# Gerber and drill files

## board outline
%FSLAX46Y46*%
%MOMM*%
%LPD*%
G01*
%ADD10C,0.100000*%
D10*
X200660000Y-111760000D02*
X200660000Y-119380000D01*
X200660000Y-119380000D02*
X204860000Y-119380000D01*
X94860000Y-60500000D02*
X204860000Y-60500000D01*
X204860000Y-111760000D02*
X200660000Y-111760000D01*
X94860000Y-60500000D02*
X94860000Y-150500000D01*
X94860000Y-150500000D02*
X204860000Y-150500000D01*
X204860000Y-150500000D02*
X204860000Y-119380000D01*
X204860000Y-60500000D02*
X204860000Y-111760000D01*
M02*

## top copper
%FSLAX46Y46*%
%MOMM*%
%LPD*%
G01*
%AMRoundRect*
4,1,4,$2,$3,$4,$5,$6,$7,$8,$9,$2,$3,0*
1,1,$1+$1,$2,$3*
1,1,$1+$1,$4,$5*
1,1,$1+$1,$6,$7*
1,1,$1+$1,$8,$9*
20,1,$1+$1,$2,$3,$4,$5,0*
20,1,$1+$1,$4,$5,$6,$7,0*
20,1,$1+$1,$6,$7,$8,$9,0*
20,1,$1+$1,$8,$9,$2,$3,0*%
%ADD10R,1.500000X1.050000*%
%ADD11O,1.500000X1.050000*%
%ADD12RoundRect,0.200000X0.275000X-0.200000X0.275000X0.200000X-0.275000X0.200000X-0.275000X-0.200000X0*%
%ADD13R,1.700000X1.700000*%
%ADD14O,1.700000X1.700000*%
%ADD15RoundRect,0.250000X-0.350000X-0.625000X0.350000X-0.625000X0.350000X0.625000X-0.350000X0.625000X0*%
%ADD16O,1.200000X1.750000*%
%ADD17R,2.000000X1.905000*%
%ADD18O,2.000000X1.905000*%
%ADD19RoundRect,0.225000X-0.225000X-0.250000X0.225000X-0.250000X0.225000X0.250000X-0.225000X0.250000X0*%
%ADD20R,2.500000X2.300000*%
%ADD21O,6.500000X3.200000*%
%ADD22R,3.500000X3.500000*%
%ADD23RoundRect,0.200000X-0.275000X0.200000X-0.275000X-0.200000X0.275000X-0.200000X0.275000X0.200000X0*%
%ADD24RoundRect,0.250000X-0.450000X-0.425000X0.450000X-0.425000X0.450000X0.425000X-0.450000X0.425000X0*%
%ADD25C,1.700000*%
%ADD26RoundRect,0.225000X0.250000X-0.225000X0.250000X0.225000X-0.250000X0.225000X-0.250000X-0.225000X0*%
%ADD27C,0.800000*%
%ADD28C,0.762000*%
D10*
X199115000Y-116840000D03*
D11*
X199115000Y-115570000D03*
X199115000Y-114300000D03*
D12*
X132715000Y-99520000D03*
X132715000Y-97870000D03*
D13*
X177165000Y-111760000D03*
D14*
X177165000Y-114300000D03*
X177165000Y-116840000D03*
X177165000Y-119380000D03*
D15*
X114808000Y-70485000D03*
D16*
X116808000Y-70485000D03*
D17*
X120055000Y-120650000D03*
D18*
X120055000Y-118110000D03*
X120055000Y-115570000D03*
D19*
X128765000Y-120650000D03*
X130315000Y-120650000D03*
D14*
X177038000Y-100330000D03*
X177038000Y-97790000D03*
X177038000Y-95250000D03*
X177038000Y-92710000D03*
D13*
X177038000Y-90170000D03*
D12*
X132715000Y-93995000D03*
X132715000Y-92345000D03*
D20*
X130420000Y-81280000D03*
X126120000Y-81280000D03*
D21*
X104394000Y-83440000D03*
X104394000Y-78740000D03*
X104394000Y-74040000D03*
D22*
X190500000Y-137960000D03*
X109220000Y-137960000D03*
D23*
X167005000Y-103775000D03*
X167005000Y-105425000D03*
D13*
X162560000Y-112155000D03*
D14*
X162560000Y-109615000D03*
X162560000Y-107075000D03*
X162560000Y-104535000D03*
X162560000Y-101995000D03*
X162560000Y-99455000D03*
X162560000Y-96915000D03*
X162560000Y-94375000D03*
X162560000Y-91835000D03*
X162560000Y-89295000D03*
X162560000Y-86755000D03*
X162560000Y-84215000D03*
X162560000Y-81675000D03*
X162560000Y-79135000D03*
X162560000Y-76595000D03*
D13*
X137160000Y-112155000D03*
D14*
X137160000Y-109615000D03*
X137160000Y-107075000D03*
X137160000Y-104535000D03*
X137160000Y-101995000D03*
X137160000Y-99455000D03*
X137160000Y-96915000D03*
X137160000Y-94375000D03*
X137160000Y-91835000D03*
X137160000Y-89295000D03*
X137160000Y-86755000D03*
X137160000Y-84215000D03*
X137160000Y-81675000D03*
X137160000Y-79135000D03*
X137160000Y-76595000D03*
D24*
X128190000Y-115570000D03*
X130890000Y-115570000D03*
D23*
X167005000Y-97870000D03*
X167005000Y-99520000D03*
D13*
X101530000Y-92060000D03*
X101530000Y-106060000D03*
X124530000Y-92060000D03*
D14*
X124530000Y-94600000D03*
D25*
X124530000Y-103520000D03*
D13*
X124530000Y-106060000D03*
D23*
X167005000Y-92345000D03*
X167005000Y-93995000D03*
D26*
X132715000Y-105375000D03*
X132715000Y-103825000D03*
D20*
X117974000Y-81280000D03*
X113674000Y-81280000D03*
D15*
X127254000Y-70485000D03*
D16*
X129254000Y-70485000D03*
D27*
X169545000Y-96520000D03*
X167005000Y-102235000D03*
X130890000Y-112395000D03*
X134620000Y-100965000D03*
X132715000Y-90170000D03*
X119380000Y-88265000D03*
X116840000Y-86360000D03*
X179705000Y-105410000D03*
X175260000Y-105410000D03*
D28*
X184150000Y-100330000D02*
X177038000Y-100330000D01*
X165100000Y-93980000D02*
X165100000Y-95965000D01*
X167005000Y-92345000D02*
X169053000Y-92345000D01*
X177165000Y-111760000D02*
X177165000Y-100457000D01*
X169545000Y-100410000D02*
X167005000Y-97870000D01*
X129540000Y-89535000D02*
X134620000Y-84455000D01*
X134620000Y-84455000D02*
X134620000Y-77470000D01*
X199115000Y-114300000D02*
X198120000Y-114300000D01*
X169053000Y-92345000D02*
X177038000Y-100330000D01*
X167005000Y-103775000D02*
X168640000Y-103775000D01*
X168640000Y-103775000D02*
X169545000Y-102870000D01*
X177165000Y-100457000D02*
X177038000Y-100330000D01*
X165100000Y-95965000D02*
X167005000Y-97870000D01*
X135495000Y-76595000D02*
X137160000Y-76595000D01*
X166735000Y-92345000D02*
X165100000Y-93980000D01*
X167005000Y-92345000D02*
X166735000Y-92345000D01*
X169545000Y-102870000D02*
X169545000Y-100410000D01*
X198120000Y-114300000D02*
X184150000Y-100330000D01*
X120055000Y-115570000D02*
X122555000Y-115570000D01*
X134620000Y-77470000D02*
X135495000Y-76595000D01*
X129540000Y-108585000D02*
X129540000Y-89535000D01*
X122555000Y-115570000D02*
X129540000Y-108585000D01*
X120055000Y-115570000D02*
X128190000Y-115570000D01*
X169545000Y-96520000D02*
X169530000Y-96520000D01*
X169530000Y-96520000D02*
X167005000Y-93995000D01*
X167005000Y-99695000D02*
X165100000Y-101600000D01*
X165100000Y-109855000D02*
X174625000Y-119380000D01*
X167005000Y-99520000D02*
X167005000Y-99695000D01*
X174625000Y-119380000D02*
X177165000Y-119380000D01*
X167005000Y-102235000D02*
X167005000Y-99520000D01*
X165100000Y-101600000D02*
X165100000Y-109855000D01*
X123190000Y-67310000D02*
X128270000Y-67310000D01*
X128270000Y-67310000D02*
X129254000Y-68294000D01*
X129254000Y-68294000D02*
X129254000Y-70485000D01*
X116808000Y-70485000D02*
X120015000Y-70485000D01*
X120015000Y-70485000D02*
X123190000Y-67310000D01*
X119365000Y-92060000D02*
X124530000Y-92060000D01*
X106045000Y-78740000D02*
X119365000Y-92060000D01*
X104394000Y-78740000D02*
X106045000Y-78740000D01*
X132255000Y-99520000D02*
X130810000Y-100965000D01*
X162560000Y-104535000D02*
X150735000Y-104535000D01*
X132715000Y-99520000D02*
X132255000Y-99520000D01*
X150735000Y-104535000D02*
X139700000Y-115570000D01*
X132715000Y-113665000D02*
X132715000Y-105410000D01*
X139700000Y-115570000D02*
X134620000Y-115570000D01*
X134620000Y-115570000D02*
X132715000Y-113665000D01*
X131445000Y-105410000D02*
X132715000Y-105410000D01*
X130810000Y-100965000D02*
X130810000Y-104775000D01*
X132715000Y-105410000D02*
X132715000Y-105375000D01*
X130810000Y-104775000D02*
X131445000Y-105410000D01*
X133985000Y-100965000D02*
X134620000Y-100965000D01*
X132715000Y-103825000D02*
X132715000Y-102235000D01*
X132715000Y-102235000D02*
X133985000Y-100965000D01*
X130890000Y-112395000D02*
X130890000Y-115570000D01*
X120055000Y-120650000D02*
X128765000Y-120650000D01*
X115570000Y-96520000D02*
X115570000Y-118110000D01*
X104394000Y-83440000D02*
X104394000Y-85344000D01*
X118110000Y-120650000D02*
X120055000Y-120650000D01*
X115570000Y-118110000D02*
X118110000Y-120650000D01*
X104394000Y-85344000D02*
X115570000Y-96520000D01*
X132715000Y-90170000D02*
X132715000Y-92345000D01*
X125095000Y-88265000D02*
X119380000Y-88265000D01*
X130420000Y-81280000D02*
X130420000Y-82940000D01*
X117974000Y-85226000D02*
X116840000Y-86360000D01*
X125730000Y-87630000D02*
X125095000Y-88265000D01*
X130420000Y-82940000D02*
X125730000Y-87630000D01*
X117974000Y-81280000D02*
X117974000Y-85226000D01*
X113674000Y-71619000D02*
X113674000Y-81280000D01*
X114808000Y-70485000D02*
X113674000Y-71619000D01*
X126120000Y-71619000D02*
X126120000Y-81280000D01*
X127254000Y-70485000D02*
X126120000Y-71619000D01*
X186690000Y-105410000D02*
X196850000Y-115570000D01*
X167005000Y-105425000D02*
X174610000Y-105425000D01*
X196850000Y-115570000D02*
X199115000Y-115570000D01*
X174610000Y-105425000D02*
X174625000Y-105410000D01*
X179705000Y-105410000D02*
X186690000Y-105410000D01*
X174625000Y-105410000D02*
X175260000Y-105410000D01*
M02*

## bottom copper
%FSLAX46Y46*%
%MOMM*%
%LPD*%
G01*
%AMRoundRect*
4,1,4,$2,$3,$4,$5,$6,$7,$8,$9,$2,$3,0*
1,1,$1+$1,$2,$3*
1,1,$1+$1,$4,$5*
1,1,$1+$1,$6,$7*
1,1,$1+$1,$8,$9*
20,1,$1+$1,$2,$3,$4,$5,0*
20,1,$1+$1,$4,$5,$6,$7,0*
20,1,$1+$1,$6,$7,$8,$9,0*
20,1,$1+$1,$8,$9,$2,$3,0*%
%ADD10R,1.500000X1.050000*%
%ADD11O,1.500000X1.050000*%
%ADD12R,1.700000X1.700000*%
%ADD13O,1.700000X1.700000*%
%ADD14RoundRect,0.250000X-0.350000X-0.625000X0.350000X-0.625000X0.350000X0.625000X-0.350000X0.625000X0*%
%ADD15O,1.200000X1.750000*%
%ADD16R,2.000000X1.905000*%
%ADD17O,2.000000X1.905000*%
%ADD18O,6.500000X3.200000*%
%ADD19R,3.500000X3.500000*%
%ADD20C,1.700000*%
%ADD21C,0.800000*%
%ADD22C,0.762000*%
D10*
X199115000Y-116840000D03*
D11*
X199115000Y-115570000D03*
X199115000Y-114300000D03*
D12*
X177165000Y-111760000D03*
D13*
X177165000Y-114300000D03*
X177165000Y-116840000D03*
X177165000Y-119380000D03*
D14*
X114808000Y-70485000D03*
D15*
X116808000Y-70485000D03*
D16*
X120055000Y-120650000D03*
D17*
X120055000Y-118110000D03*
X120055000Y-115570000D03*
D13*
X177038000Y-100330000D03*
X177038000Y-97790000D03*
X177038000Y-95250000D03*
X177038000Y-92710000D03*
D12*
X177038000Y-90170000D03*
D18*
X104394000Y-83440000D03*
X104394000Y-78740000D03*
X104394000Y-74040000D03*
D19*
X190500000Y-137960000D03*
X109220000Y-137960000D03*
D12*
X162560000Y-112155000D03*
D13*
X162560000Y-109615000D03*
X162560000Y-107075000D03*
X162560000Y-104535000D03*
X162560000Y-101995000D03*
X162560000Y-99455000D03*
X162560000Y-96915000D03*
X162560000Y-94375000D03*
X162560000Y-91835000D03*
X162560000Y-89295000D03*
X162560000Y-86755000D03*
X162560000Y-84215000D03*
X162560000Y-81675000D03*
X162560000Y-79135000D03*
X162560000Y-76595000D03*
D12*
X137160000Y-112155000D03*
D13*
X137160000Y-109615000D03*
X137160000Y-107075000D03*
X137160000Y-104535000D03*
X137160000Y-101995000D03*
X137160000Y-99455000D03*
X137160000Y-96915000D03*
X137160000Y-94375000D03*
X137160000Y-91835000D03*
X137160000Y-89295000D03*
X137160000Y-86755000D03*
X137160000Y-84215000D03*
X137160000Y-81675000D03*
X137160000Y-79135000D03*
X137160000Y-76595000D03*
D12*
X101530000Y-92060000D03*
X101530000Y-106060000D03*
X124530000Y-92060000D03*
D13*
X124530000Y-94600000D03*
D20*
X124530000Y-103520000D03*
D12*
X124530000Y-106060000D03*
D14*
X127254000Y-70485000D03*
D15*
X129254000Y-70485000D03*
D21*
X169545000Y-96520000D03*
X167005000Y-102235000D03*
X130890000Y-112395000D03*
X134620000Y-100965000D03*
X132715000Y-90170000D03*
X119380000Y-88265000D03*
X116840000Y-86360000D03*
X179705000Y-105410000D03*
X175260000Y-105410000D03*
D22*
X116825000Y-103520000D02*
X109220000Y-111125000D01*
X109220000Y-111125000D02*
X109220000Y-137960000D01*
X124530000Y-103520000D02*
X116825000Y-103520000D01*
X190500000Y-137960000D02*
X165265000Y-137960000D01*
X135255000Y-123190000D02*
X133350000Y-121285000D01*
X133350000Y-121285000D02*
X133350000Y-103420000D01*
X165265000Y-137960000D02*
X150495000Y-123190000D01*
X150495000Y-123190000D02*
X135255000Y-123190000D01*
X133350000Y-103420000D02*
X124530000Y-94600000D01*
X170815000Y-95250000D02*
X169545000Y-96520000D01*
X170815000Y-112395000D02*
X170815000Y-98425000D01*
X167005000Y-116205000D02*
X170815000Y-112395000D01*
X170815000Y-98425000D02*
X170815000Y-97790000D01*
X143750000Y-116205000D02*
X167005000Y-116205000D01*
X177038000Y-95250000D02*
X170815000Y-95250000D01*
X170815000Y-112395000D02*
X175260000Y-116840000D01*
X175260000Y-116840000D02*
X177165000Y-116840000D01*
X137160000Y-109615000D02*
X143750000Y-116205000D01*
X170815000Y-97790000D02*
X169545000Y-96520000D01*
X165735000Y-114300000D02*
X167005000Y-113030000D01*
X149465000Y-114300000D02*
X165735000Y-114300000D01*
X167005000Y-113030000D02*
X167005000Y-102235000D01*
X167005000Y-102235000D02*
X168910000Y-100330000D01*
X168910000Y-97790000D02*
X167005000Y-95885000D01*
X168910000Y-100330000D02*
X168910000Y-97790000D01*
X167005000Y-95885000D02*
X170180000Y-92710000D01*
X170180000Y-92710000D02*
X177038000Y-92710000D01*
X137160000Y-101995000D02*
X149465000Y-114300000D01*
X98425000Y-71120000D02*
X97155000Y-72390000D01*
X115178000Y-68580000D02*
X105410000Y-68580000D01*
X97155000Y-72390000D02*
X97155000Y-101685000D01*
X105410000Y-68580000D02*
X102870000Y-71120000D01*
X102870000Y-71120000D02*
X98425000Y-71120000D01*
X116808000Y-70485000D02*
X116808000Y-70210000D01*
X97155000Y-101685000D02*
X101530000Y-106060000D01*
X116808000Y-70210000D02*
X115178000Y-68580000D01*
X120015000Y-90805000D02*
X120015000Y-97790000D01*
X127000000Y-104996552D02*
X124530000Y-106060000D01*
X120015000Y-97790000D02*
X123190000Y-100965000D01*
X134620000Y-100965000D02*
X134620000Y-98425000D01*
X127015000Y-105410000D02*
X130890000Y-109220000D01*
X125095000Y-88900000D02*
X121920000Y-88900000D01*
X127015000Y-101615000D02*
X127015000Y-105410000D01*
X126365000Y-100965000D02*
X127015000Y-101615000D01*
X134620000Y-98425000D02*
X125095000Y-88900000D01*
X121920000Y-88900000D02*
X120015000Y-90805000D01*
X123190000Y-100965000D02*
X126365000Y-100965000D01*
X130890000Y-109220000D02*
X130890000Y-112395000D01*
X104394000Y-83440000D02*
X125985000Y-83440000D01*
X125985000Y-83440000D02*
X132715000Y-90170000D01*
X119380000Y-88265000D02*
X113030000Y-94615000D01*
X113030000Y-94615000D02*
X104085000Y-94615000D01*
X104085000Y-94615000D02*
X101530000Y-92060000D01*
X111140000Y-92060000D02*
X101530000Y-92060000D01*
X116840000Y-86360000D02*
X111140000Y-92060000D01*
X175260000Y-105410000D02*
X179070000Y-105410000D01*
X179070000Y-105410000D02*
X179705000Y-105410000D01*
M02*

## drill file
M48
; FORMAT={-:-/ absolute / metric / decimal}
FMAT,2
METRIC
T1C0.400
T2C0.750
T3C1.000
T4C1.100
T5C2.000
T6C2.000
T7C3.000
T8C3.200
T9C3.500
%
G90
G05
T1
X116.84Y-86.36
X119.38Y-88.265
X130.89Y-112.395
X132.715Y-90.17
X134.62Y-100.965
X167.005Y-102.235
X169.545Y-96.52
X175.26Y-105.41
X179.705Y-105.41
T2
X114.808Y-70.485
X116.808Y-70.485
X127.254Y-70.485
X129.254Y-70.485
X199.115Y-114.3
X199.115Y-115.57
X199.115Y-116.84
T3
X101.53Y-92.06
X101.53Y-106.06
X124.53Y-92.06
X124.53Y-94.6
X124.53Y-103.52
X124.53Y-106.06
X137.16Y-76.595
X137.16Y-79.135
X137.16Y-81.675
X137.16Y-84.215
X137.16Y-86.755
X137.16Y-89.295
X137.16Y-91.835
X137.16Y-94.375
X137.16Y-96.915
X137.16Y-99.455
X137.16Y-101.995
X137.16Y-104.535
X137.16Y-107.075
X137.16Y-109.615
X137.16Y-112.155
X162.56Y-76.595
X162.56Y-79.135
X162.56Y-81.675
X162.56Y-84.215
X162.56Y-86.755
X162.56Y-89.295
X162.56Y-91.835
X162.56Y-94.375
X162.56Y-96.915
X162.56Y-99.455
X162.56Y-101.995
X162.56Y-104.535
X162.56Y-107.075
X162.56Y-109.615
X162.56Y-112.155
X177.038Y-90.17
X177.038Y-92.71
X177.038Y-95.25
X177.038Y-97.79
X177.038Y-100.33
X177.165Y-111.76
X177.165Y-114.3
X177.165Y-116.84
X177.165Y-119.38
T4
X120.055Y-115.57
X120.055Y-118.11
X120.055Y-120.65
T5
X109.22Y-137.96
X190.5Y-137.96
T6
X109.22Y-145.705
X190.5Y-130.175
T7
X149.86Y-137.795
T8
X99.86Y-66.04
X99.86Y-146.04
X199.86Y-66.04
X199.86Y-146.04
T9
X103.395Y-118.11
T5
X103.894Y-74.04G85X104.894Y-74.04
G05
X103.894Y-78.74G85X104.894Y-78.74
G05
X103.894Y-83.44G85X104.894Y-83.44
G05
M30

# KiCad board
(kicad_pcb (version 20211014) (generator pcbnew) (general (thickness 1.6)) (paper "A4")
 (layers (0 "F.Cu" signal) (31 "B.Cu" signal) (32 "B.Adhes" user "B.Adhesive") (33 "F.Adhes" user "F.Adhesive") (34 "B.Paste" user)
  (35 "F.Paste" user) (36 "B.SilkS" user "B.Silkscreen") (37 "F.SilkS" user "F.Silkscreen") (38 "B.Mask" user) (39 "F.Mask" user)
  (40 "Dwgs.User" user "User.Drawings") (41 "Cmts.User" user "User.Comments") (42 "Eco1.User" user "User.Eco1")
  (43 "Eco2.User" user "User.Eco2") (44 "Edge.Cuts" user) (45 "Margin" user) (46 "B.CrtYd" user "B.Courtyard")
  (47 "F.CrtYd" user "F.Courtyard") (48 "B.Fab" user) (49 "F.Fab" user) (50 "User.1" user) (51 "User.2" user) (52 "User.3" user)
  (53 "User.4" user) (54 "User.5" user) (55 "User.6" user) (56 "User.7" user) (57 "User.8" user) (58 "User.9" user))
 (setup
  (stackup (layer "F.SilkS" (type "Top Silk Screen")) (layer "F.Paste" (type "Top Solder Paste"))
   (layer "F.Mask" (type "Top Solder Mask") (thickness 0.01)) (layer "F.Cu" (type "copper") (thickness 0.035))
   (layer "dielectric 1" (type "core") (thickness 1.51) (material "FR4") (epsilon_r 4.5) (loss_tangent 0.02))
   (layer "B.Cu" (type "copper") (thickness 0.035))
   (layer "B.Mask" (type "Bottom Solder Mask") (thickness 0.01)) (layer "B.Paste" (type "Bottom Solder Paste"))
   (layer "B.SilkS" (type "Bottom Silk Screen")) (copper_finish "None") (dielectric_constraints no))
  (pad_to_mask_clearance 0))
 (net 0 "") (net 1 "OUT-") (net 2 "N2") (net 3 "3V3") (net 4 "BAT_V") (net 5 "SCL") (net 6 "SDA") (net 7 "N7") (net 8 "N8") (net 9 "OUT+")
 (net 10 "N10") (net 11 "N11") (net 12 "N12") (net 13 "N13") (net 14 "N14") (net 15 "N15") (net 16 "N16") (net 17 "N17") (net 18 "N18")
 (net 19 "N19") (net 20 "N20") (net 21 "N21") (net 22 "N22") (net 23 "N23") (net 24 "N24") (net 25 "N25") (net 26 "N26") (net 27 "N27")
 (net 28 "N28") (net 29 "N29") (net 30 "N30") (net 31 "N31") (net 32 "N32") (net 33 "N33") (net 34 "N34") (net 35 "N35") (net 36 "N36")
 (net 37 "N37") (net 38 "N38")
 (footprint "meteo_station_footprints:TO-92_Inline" (layer "F.Cu") (at 199.115 116.84 90)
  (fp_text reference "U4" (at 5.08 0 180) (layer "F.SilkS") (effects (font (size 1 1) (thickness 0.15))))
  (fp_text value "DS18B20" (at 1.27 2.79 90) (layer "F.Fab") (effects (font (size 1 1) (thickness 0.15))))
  (pad "1" thru_hole rect (at 0 0 90) (size 1.05 1.5) (drill 0.75) (layers *.Cu *.Mask) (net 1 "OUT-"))
  (pad "2" thru_hole oval (at 1.27 0 90) (size 1.05 1.5) (drill 0.75) (layers *.Cu *.Mask) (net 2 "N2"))
  (pad "3" thru_hole oval (at 2.54 0 90) (size 1.05 1.5) (drill 0.75) (layers *.Cu *.Mask) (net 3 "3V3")))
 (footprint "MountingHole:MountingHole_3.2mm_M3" (layer "F.Cu") (at 199.86 146.04)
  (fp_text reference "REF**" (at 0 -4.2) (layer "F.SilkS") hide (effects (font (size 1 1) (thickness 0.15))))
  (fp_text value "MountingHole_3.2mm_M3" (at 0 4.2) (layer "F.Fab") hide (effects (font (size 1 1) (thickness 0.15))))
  (pad "" np_thru_hole circle locked (at 0 0) (size 3.2 3.2) (drill 3.2) (layers *.Cu *.Mask)))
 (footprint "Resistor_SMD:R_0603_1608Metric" (layer "F.Cu") (at 132.715 98.695 90)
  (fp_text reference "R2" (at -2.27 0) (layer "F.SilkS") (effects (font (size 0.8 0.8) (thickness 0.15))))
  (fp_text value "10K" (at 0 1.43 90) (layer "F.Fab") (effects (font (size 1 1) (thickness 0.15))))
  (pad "1" smd roundrect locked (at -0.825 0 90) (size 0.8 0.95) (layers "F.Cu" "F.Paste" "F.Mask") (roundrect_rratio 0.25) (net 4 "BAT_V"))
  (pad "2" smd roundrect locked (at 0.825 0 90) (size 0.8 0.95) (layers "F.Cu" "F.Paste" "F.Mask") (roundrect_rratio 0.25) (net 1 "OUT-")))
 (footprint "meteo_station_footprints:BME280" (layer "F.Cu") (at 182.245 115.57)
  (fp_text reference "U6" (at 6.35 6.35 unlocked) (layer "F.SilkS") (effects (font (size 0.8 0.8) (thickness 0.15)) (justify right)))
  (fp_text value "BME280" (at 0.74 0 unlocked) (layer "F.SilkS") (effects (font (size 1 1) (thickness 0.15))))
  (pad "1" thru_hole rect (at -5.08 -3.81) (size 1.7 1.7) (drill 1) (layers *.Cu *.Mask "B.SilkS") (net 3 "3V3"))
  (pad "2" thru_hole oval (at -5.08 -1.27) (size 1.7 1.7) (drill 1) (layers *.Cu *.Mask) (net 1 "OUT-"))
  (pad "3" thru_hole oval (at -5.08 1.27) (size 1.7 1.7) (drill 1) (layers *.Cu *.Mask) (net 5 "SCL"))
  (pad "4" thru_hole oval (at -5.08 3.81) (size 1.7 1.7) (drill 1) (layers *.Cu *.Mask) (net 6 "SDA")))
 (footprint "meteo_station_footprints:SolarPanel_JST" (layer "F.Cu") (at 115.824 71.12)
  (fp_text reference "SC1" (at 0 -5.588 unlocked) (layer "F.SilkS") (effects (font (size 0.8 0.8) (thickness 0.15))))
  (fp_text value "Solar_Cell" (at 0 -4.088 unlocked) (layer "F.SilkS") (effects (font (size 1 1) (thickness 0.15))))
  (pad "1" thru_hole roundrect (at -1.016 -0.635) (size 1.2 1.75) (drill 0.75) (layers *.Cu *.Mask) (roundrect_rratio 0.208333) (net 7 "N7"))
  (pad "2" thru_hole oval (at 0.984 -0.635) (size 1.2 1.75) (drill 0.75) (layers *.Cu *.Mask) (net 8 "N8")))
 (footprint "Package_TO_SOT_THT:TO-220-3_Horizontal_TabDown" (layer "F.Cu") (at 120.055 120.65 90)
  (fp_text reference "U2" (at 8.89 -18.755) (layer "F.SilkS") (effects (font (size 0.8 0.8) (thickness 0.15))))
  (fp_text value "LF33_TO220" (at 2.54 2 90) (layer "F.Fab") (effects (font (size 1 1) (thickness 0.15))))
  (pad "" np_thru_hole oval locked (at 2.54 -16.66 90) (size 3.5 3.5) (drill 3.5) (layers *.Cu *.Mask))
  (pad "1" thru_hole rect locked (at 0 0 90) (size 1.905 2) (drill 1.1) (layers *.Cu *.Mask) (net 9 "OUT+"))
  (pad "2" thru_hole oval locked (at 2.54 0 90) (size 1.905 2) (drill 1.1) (layers *.Cu *.Mask) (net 1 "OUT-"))
  (pad "3" thru_hole oval locked (at 5.08 0 90) (size 1.905 2) (drill 1.1) (layers *.Cu *.Mask) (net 3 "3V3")))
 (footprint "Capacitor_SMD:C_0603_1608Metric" (layer "F.Cu") (at 129.54 120.65)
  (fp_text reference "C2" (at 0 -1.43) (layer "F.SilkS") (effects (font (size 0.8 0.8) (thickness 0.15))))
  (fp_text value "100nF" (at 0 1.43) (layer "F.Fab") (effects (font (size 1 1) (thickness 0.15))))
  (pad "1" smd roundrect locked (at -0.775 0) (size 0.9 0.95) (layers "F.Cu" "F.Paste" "F.Mask") (roundrect_rratio 0.25) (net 9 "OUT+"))
  (pad "2" smd roundrect locked (at 0.775 0) (size 0.9 0.95) (layers "F.Cu" "F.Paste" "F.Mask") (roundrect_rratio 0.25) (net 1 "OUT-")))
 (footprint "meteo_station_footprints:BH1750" (layer "F.Cu") (at 184.15 95.25)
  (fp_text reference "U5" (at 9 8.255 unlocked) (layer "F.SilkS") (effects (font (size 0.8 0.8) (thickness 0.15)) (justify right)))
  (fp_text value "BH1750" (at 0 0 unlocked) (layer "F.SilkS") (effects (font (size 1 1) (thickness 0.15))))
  (pad "1" thru_hole oval (at -7.112 5.08) (size 1.7 1.7) (drill 1) (layers *.Cu *.Mask) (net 3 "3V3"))
  (pad "2" thru_hole oval (at -7.112 2.54) (size 1.7 1.7) (drill 1) (layers *.Cu *.Mask) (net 1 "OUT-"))
  (pad "3" thru_hole oval (at -7.112 0) (size 1.7 1.7) (drill 1) (layers *.Cu *.Mask) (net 5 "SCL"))
  (pad "4" thru_hole oval (at -7.112 -2.54) (size 1.7 1.7) (drill 1) (layers *.Cu *.Mask) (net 6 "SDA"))
  (pad "5" thru_hole rect (at -7.112 -5.08) (size 1.7 1.7) (drill 1) (layers *.Cu *.Mask) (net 1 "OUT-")))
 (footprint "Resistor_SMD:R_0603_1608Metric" (layer "F.Cu") (at 132.715 93.17 90)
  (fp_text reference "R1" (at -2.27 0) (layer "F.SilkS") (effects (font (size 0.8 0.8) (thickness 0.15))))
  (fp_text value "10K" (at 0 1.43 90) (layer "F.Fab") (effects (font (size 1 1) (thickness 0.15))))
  (pad "1" smd roundrect locked (at -0.825 0 90) (size 0.8 0.95) (layers "F.Cu" "F.Paste" "F.Mask") (roundrect_rratio 0.25) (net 4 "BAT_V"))
  (pad "2" smd roundrect locked (at 0.825 0 90) (size 0.8 0.95) (layers "F.Cu" "F.Paste" "F.Mask") (roundrect_rratio 0.25) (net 9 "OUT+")))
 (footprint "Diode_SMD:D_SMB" (layer "F.Cu") (at 128.27 81.28 180)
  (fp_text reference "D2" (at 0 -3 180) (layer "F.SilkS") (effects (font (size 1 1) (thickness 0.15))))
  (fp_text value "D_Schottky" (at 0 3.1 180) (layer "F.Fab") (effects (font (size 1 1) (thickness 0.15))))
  (pad "1" smd rect locked (at -2.15 0 180) (size 2.5 2.3) (layers "F.Cu" "F.Paste" "F.Mask") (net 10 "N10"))
  (pad "2" smd rect locked (at 2.15 0 180) (size 2.5 2.3) (layers "F.Cu" "F.Paste" "F.Mask") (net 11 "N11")))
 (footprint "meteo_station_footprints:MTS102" (layer "F.Cu") (at 104.394 78.74 90)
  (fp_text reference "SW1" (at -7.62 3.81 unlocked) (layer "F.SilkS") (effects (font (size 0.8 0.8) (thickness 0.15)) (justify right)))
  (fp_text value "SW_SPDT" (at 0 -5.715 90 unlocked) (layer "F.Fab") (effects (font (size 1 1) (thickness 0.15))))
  (pad "1" thru_hole oval (at -4.7 0 90) (size 3.2 6.5) (drill oval 2 3) (layers *.Cu *.Mask) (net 9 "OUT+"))
  (pad "2" thru_hole oval (at 0 0 90) (size 3.2 6.5) (drill oval 2 3) (layers *.Cu *.Mask) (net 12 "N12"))
  (pad "3" thru_hole oval (at 4.7 0 90) (size 3.2 6.5) (drill oval 2 3) (layers *.Cu *.Mask) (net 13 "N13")))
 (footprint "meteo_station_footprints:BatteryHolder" (layer "F.Cu") (at 149.86 137.795)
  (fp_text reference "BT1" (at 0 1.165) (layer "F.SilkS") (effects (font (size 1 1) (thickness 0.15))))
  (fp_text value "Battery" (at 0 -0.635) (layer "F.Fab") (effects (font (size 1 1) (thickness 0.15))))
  (pad "" np_thru_hole circle (at 0 0) (size 3 3) (drill 3) (layers *.Cu *.Mask))
  (pad "" np_thru_hole circle (at 40.64 -7.62) (size 2 2) (drill 2) (layers *.Cu *.Mask))
  (pad "" np_thru_hole circle (at -40.64 7.91) (size 2 2) (drill 2) (layers *.Cu *.Mask))
  (pad "1" thru_hole rect (at 40.64 0.165) (size 3.5 3.5) (drill 2) (layers *.Cu *.Mask) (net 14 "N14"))
  (pad "2" thru_hole rect (at -40.64 0.165) (size 3.5 3.5) (drill 2) (layers *.Cu *.Mask) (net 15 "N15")))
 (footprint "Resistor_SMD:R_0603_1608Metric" (layer "F.Cu") (at 167.005 104.6 -90)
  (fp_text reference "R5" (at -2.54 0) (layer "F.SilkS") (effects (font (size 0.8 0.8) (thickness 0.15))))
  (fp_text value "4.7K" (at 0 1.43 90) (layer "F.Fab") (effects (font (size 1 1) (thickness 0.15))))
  (pad "1" smd roundrect locked (at -0.825 0 270) (size 0.8 0.95) (layers "F.Cu" "F.Paste" "F.Mask") (roundrect_rratio 0.25) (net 3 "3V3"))
  (pad "2" smd roundrect locked (at 0.825 0 270) (size 0.8 0.95) (layers "F.Cu" "F.Paste" "F.Mask") (roundrect_rratio 0.25) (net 2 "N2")))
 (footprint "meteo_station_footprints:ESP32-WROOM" (layer "F.Cu") (at 149.86 93.11 180)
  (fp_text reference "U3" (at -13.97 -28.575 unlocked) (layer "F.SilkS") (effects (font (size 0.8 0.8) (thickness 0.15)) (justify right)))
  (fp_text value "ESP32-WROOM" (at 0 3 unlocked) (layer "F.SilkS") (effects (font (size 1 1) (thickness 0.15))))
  (pad "1" thru_hole rect (at -12.7 -19.045 180) (size 1.7 1.7) (drill 1) (layers *.Cu *.Mask) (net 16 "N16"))
  (pad "2" thru_hole oval (at -12.7 -16.505 180) (size 1.7 1.7) (drill 1) (layers *.Cu *.Mask) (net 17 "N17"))
  (pad "3" thru_hole oval (at -12.7 -13.965 180) (size 1.7 1.7) (drill 1) (layers *.Cu *.Mask) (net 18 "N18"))
  (pad "4" thru_hole oval (at -12.7 -11.425 180) (size 1.7 1.7) (drill 1) (layers *.Cu *.Mask) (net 4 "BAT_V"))
  (pad "5" thru_hole oval (at -12.7 -8.885 180) (size 1.7 1.7) (drill 1) (layers *.Cu *.Mask) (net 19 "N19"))
  (pad "6" thru_hole oval (at -12.7 -6.345 180) (size 1.7 1.7) (drill 1) (layers *.Cu *.Mask) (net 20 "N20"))
  (pad "7" thru_hole oval (at -12.7 -3.805 180) (size 1.7 1.7) (drill 1) (layers *.Cu *.Mask) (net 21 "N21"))
  (pad "8" thru_hole oval (at -12.7 -1.265 180) (size 1.7 1.7) (drill 1) (layers *.Cu *.Mask) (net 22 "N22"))
  (pad "9" thru_hole oval (at -12.7 1.275 180) (size 1.7 1.7) (drill 1) (layers *.Cu *.Mask) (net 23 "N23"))
  (pad "10" thru_hole oval (at -12.7 3.815 180) (size 1.7 1.7) (drill 1) (layers *.Cu *.Mask) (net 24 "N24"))
  (pad "11" thru_hole oval (at -12.7 6.355 180) (size 1.7 1.7) (drill 1) (layers *.Cu *.Mask) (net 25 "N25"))
  (pad "12" thru_hole oval (at -12.7 8.895 180) (size 1.7 1.7) (drill 1) (layers *.Cu *.Mask) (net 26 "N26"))
  (pad "13" thru_hole oval (at -12.7 11.435 180) (size 1.7 1.7) (drill 1) (layers *.Cu *.Mask) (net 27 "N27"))
  (pad "14" thru_hole oval (at -12.7 13.975 180) (size 1.7 1.7) (drill 1) (layers *.Cu *.Mask) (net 1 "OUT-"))
  (pad "15" thru_hole oval (at -12.7 16.515 180) (size 1.7 1.7) (drill 1) (layers *.Cu *.Mask) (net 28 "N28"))
  (pad "16" thru_hole rect (at 12.7 -19.045 180) (size 1.7 1.7) (drill 1) (layers *.Cu *.Mask) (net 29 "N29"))
  (pad "17" thru_hole oval (at 12.7 -16.505 180) (size 1.7 1.7) (drill 1) (layers *.Cu *.Mask) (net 5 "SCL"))
  (pad "18" thru_hole oval (at 12.7 -13.965 180) (size 1.7 1.7) (drill 1) (layers *.Cu *.Mask) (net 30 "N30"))
  (pad "19" thru_hole oval (at 12.7 -11.425 180) (size 1.7 1.7) (drill 1) (layers *.Cu *.Mask) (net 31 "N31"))
  (pad "20" thru_hole oval (at 12.7 -8.885 180) (size 1.7 1.7) (drill 1) (layers *.Cu *.Mask) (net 6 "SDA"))
  (pad "21" thru_hole oval (at 12.7 -6.345 180) (size 1.7 1.7) (drill 1) (layers *.Cu *.Mask) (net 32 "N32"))
  (pad "22" thru_hole oval (at 12.7 -3.805 180) (size 1.7 1.7) (drill 1) (layers *.Cu *.Mask) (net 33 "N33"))
  (pad "23" thru_hole oval (at 12.7 -1.265 180) (size 1.7 1.7) (drill 1) (layers *.Cu *.Mask) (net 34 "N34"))
  (pad "24" thru_hole oval (at 12.7 1.275 180) (size 1.7 1.7) (drill 1) (layers *.Cu *.Mask) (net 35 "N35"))
  (pad "25" thru_hole oval (at 12.7 3.815 180) (size 1.7 1.7) (drill 1) (layers *.Cu *.Mask) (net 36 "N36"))
  (pad "26" thru_hole oval (at 12.7 6.355 180) (size 1.7 1.7) (drill 1) (layers *.Cu *.Mask) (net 2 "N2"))
  (pad "27" thru_hole oval (at 12.7 8.895 180) (size 1.7 1.7) (drill 1) (layers *.Cu *.Mask) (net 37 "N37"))
  (pad "28" thru_hole oval (at 12.7 11.435 180) (size 1.7 1.7) (drill 1) (layers *.Cu *.Mask) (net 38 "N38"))
  (pad "29" thru_hole oval (at 12.7 13.975 180) (size 1.7 1.7) (drill 1) (layers *.Cu *.Mask) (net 1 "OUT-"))
  (pad "30" thru_hole oval (at 12.7 16.515 180) (size 1.7 1.7) (drill 1) (layers *.Cu *.Mask) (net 3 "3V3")))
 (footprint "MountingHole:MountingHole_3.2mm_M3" (layer "F.Cu") (at 99.86 146.04)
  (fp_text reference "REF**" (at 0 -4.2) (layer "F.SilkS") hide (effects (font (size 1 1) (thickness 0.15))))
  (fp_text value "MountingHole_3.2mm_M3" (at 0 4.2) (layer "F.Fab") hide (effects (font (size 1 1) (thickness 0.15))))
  (pad "" np_thru_hole circle locked (at 0 0) (size 3.2 3.2) (drill 3.2) (layers *.Cu *.Mask)))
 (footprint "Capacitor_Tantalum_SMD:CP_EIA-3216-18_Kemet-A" (layer "F.Cu") (at 129.54 115.57)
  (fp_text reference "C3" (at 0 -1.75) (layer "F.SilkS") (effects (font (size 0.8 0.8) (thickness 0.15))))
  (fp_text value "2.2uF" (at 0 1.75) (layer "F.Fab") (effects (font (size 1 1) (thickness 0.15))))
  (pad "1" smd roundrect locked (at -1.35 0) (size 1.4 1.35) (layers "F.Cu" "F.Paste" "F.Mask") (roundrect_rratio 0.185185) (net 3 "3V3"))
  (pad "2" smd roundrect locked (at 1.35 0) (size 1.4 1.35) (layers "F.Cu" "F.Paste" "F.Mask") (roundrect_rratio 0.185185) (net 1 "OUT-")))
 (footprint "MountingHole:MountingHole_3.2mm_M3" (layer "F.Cu") (at 199.86 66.04)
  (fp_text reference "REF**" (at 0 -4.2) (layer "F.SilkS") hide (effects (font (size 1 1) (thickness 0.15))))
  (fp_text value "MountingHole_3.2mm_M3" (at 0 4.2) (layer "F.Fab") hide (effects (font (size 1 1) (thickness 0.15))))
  (pad "" np_thru_hole circle locked (at 0 0) (size 3.2 3.2) (drill 3.2) (layers *.Cu *.Mask)))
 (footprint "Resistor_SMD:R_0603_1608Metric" (layer "F.Cu") (at 167.005 98.695 -90)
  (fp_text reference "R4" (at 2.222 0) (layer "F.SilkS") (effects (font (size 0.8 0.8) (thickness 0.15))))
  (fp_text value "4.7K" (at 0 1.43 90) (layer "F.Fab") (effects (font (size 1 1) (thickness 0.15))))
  (pad "1" smd roundrect locked (at -0.825 0 270) (size 0.8 0.95) (layers "F.Cu" "F.Paste" "F.Mask") (roundrect_rratio 0.25) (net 3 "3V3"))
  (pad "2" smd roundrect locked (at 0.825 0 270) (size 0.8 0.95) (layers "F.Cu" "F.Paste" "F.Mask") (roundrect_rratio 0.25) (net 6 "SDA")))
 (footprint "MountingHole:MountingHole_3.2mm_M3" (layer "F.Cu") (at 99.86 66.04)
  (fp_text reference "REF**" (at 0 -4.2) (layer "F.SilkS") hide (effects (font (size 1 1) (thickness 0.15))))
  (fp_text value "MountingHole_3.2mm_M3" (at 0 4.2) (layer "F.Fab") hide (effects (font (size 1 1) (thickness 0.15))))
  (pad "" np_thru_hole circle locked (at 0 0) (size 3.2 3.2) (drill 3.2) (layers *.Cu *.Mask)))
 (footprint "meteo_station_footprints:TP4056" (layer "F.Cu") (at 113.03 99.06)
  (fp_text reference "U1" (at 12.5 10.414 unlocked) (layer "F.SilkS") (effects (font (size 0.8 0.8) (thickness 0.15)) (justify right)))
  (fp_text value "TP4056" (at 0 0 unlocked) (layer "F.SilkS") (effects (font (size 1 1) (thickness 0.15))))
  (pad "1" thru_hole rect (at -11.5 -7) (size 1.7 1.7) (drill 1) (layers *.Cu *.Mask) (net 10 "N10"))
  (pad "2" thru_hole rect (at -11.5 7) (size 1.7 1.7) (drill 1) (layers *.Cu *.Mask) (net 8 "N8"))
  (pad "3" thru_hole rect (at 11.5 -7) (size 1.7 1.7) (drill 1) (layers *.Cu *.Mask) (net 12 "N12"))
  (pad "4" thru_hole oval (at 11.5 -4.46) (size 1.7 1.7) (drill 1) (layers *.Cu *.Mask) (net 14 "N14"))
  (pad "5" thru_hole circle (at 11.5 4.46) (size 1.7 1.7) (drill 1) (layers *.Cu *.Mask) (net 15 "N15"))
  (pad "6" thru_hole rect (at 11.5 7) (size 1.7 1.7) (drill 1) (layers *.Cu *.Mask) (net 1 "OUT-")))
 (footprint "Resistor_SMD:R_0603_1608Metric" (layer "F.Cu") (at 167.005 93.17 -90)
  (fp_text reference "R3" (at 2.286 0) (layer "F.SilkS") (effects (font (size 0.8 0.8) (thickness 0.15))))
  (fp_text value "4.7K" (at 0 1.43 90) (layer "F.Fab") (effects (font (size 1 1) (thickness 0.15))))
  (pad "1" smd roundrect locked (at -0.825 0 270) (size 0.8 0.95) (layers "F.Cu" "F.Paste" "F.Mask") (roundrect_rratio 0.25) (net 3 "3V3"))
  (pad "2" smd roundrect locked (at 0.825 0 270) (size 0.8 0.95) (layers "F.Cu" "F.Paste" "F.Mask") (roundrect_rratio 0.25) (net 5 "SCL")))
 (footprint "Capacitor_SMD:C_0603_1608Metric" (layer "F.Cu") (at 132.715 104.6 90)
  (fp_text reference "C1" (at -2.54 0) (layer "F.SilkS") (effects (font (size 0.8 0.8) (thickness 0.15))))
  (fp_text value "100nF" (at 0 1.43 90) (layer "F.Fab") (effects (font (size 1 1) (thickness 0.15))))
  (pad "1" smd roundrect locked (at -0.775 0 90) (size 0.9 0.95) (layers "F.Cu" "F.Paste" "F.Mask") (roundrect_rratio 0.25) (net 4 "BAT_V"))
  (pad "2" smd roundrect locked (at 0.775 0 90) (size 0.9 0.95) (layers "F.Cu" "F.Paste" "F.Mask") (roundrect_rratio 0.25) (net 1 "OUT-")))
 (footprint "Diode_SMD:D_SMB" (layer "F.Cu") (at 115.824 81.28 180)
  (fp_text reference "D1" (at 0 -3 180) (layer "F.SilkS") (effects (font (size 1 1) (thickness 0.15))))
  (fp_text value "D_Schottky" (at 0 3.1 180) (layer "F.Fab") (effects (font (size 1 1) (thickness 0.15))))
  (pad "1" smd rect locked (at -2.15 0 180) (size 2.5 2.3) (layers "F.Cu" "F.Paste" "F.Mask") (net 10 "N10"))
  (pad "2" smd rect locked (at 2.15 0 180) (size 2.5 2.3) (layers "F.Cu" "F.Paste" "F.Mask") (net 7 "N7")))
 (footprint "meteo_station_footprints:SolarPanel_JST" (layer "F.Cu") (at 128.27 71.12)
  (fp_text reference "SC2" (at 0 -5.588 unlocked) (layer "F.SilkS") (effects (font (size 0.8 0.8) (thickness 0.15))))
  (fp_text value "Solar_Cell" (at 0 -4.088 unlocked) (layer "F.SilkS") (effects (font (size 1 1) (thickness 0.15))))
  (pad "1" thru_hole roundrect (at -1.016 -0.635) (size 1.2 1.75) (drill 0.75) (layers *.Cu *.Mask) (roundrect_rratio 0.208333)
   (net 11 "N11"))
  (pad "2" thru_hole oval (at 0.984 -0.635) (size 1.2 1.75) (drill 0.75) (layers *.Cu *.Mask) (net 8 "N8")))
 (gr_line (start 200.66 111.76) (end 200.66 119.38) (layer "Edge.Cuts") (width 0.1))
 (gr_line (start 200.66 119.38) (end 204.86 119.38) (layer "Edge.Cuts") (width 0.1))
 (gr_line (start 94.86 60.5) (end 204.86 60.5) (layer "Edge.Cuts") (width 0.1))
 (gr_line (start 204.86 111.76) (end 200.66 111.76) (layer "Edge.Cuts") (width 0.1))
 (gr_line (start 94.86 60.5) (end 94.86 150.5) (layer "Edge.Cuts") (width 0.1))
 (gr_line (start 94.86 150.5) (end 204.86 150.5) (layer "Edge.Cuts") (width 0.1))
 (gr_line (start 204.86 150.5) (end 204.86 119.38) (layer "Edge.Cuts") (width 0.1))
 (gr_line (start 204.86 60.5) (end 204.86 111.76) (layer "Edge.Cuts") (width 0.1))
 (segment (start 116.825 103.52) (end 109.22 111.125) (width 0.762) (layer "B.Cu") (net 15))
 (segment (start 109.22 111.125) (end 109.22 137.96) (width 0.762) (layer "B.Cu") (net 15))
 (segment (start 124.53 103.52) (end 116.825 103.52) (width 0.762) (layer "B.Cu") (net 15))
 (segment (start 190.5 137.96) (end 165.265 137.96) (width 0.762) (layer "B.Cu") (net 14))
 (segment (start 135.255 123.19) (end 133.35 121.285) (width 0.762) (layer "B.Cu") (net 14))
 (segment (start 133.35 121.285) (end 133.35 103.42) (width 0.762) (layer "B.Cu") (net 14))
 (segment (start 165.265 137.96) (end 150.495 123.19) (width 0.762) (layer "B.Cu") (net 14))
 (segment (start 150.495 123.19) (end 135.255 123.19) (width 0.762) (layer "B.Cu") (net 14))
 (segment (start 133.35 103.42) (end 124.53 94.6) (width 0.762) (layer "B.Cu") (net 14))
 (segment (start 184.15 100.33) (end 177.038 100.33) (width 0.762) (layer "F.Cu") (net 3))
 (segment (start 165.1 93.98) (end 165.1 95.965) (width 0.762) (layer "F.Cu") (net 3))
 (segment (start 167.005 92.345) (end 169.053 92.345) (width 0.762) (layer "F.Cu") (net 3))
 (segment (start 177.165 111.76) (end 177.165 100.457) (width 0.762) (layer "F.Cu") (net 3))
 (segment (start 169.545 100.41) (end 167.005 97.87) (width 0.762) (layer "F.Cu") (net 3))
 (segment (start 129.54 89.535) (end 134.62 84.455) (width 0.762) (layer "F.Cu") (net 3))
 (segment (start 134.62 84.455) (end 134.62 77.47) (width 0.762) (layer "F.Cu") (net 3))
 (segment (start 199.115 114.3) (end 198.12 114.3) (width 0.762) (layer "F.Cu") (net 3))
 (segment (start 169.053 92.345) (end 177.038 100.33) (width 0.762) (layer "F.Cu") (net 3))
 (segment (start 167.005 103.775) (end 168.64 103.775) (width 0.762) (layer "F.Cu") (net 3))
 (segment (start 168.64 103.775) (end 169.545 102.87) (width 0.762) (layer "F.Cu") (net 3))
 (segment (start 177.165 100.457) (end 177.038 100.33) (width 0.762) (layer "F.Cu") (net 3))
 (segment (start 165.1 95.965) (end 167.005 97.87) (width 0.762) (layer "F.Cu") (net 3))
 (segment (start 135.495 76.595) (end 137.16 76.595) (width 0.762) (layer "F.Cu") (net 3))
 (segment (start 166.735 92.345) (end 165.1 93.98) (width 0.762) (layer "F.Cu") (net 3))
 (segment (start 167.005 92.345) (end 166.735 92.345) (width 0.762) (layer "F.Cu") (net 3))
 (segment (start 169.545 102.87) (end 169.545 100.41) (width 0.762) (layer "F.Cu") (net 3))
 (segment (start 198.12 114.3) (end 184.15 100.33) (width 0.762) (layer "F.Cu") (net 3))
 (segment (start 120.055 115.57) (end 122.555 115.57) (width 0.762) (layer "F.Cu") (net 3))
 (segment (start 134.62 77.47) (end 135.495 76.595) (width 0.762) (layer "F.Cu") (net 3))
 (segment (start 129.54 108.585) (end 129.54 89.535) (width 0.762) (layer "F.Cu") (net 3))
 (segment (start 122.555 115.57) (end 129.54 108.585) (width 0.762) (layer "F.Cu") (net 3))
 (segment (start 120.055 115.57) (end 128.19 115.57) (width 0.762) (layer "F.Cu") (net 3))
 (segment (start 169.545 96.52) (end 169.53 96.52) (width 0.762) (layer "F.Cu") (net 5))
 (segment (start 169.53 96.52) (end 167.005 93.995) (width 0.762) (layer "F.Cu") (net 5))
 (via (at 169.545 96.52) (size 0.8) (drill 0.4) (layers "F.Cu" "B.Cu") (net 5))
 (segment (start 170.815 95.25) (end 169.545 96.52) (width 0.762) (layer "B.Cu") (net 5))
 (segment (start 170.815 112.395) (end 170.815 98.425) (width 0.762) (layer "B.Cu") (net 5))
 (segment (start 167.005 116.205) (end 170.815 112.395) (width 0.762) (layer "B.Cu") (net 5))
 (segment (start 170.815 98.425) (end 170.815 97.79) (width 0.762) (layer "B.Cu") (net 5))
 (segment (start 143.75 116.205) (end 167.005 116.205) (width 0.762) (layer "B.Cu") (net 5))
 (segment (start 177.038 95.25) (end 170.815 95.25) (width 0.762) (layer "B.Cu") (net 5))
 (segment (start 170.815 112.395) (end 175.26 116.84) (width 0.762) (layer "B.Cu") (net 5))
 (segment (start 175.26 116.84) (end 177.165 116.84) (width 0.762) (layer "B.Cu") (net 5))
 (segment (start 137.16 109.615) (end 143.75 116.205) (width 0.762) (layer "B.Cu") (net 5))
 (segment (start 170.815 97.79) (end 169.545 96.52) (width 0.762) (layer "B.Cu") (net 5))
 (segment (start 167.005 99.695) (end 165.1 101.6) (width 0.762) (layer "F.Cu") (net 6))
 (segment (start 165.1 109.855) (end 174.625 119.38) (width 0.762) (layer "F.Cu") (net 6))
 (segment (start 167.005 99.52) (end 167.005 99.695) (width 0.762) (layer "F.Cu") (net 6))
 (segment (start 174.625 119.38) (end 177.165 119.38) (width 0.762) (layer "F.Cu") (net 6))
 (segment (start 167.005 102.235) (end 167.005 99.52) (width 0.762) (layer "F.Cu") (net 6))
 (segment (start 165.1 101.6) (end 165.1 109.855) (width 0.762) (layer "F.Cu") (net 6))
 (via (at 167.005 102.235) (size 0.8) (drill 0.4) (layers "F.Cu" "B.Cu") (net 6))
 (segment (start 165.735 114.3) (end 167.005 113.03) (width 0.762) (layer "B.Cu") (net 6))
 (segment (start 149.465 114.3) (end 165.735 114.3) (width 0.762) (layer "B.Cu") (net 6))
 (segment (start 167.005 113.03) (end 167.005 102.235) (width 0.762) (layer "B.Cu") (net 6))
 (segment (start 167.005 102.235) (end 168.91 100.33) (width 0.762) (layer "B.Cu") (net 6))
 (segment (start 168.91 97.79) (end 167.005 95.885) (width 0.762) (layer "B.Cu") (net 6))
 (segment (start 168.91 100.33) (end 168.91 97.79) (width 0.762) (layer "B.Cu") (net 6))
 (segment (start 167.005 95.885) (end 170.18 92.71) (width 0.762) (layer "B.Cu") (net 6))
 (segment (start 170.18 92.71) (end 177.038 92.71) (width 0.762) (layer "B.Cu") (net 6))
 (segment (start 137.16 101.995) (end 149.465 114.3) (width 0.762) (layer "B.Cu") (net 6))
 (segment (start 123.19 67.31) (end 128.27 67.31) (width 0.762) (layer "F.Cu") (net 8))
 (segment (start 128.27 67.31) (end 129.254 68.294) (width 0.762) (layer "F.Cu") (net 8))
 (segment (start 129.254 68.294) (end 129.254 70.485) (width 0.762) (layer "F.Cu") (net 8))
 (segment (start 116.808 70.485) (end 120.015 70.485) (width 0.762) (layer "F.Cu") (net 8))
 (segment (start 120.015 70.485) (end 123.19 67.31) (width 0.762) (layer "F.Cu") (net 8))
 (segment (start 98.425 71.12) (end 97.155 72.39) (width 0.762) (layer "B.Cu") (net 8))
 (segment (start 115.178 68.58) (end 105.41 68.58) (width 0.762) (layer "B.Cu") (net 8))
 (segment (start 97.155 72.39) (end 97.155 101.685) (width 0.762) (layer "B.Cu") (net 8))
 (segment (start 105.41 68.58) (end 102.87 71.12) (width 0.762) (layer "B.Cu") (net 8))
 (segment (start 102.87 71.12) (end 98.425 71.12) (width 0.762) (layer "B.Cu") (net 8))
 (segment (start 116.808 70.485) (end 116.808 70.21) (width 0.762) (layer "B.Cu") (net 8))
 (segment (start 97.155 101.685) (end 101.53 106.06) (width 0.762) (layer "B.Cu") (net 8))
 (segment (start 116.808 70.21) (end 115.178 68.58) (width 0.762) (layer "B.Cu") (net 8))
 (segment (start 119.365 92.06) (end 124.53 92.06) (width 0.762) (layer "F.Cu") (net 12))
 (segment (start 106.045 78.74) (end 119.365 92.06) (width 0.762) (layer "F.Cu") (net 12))
 (segment (start 104.394 78.74) (end 106.045 78.74) (width 0.762) (layer "F.Cu") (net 12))
 (segment (start 132.255 99.52) (end 130.81 100.965) (width 0.762) (layer "F.Cu") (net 4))
 (segment (start 162.56 104.535) (end 150.735 104.535) (width 0.762) (layer "F.Cu") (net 4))
 (segment (start 132.715 99.52) (end 132.255 99.52) (width 0.762) (layer "F.Cu") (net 4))
 (segment (start 150.735 104.535) (end 139.7 115.57) (width 0.762) (layer "F.Cu") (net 4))
 (segment (start 132.715 113.665) (end 132.715 105.41) (width 0.762) (layer "F.Cu") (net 4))
 (segment (start 139.7 115.57) (end 134.62 115.57) (width 0.762) (layer "F.Cu") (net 4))
 (segment (start 134.62 115.57) (end 132.715 113.665) (width 0.762) (layer "F.Cu") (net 4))
 (segment (start 131.445 105.41) (end 132.715 105.41) (width 0.762) (layer "F.Cu") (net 4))
 (segment (start 130.81 100.965) (end 130.81 104.775) (width 0.762) (layer "F.Cu") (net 4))
 (segment (start 132.715 105.41) (end 132.715 105.375) (width 0.762) (layer "F.Cu") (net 4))
 (segment (start 130.81 104.775) (end 131.445 105.41) (width 0.762) (layer "F.Cu") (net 4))
 (segment (start 133.985 100.965) (end 134.62 100.965) (width 0.762) (layer "F.Cu") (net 1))
 (segment (start 132.715 103.825) (end 132.715 102.235) (width 0.762) (layer "F.Cu") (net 1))
 (segment (start 132.715 102.235) (end 133.985 100.965) (width 0.762) (layer "F.Cu") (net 1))
 (segment (start 130.89 112.395) (end 130.89 115.57) (width 0.762) (layer "F.Cu") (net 1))
 (via (at 130.89 112.395) (size 0.8) (drill 0.4) (layers "F.Cu" "B.Cu") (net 1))
 (via (at 134.62 100.965) (size 0.8) (drill 0.4) (layers "F.Cu" "B.Cu") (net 1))
 (segment (start 120.015 90.805) (end 120.015 97.79) (width 0.762) (layer "B.Cu") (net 1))
 (segment (start 127 104.996552) (end 124.53 106.06) (width 0.762) (layer "B.Cu") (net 1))
 (segment (start 120.015 97.79) (end 123.19 100.965) (width 0.762) (layer "B.Cu") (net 1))
 (segment (start 134.62 100.965) (end 134.62 98.425) (width 0.762) (layer "B.Cu") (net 1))
 (segment (start 127.015 105.41) (end 130.89 109.22) (width 0.762) (layer "B.Cu") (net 1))
 (segment (start 125.095 88.9) (end 121.92 88.9) (width 0.762) (layer "B.Cu") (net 1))
 (segment (start 127.015 101.615) (end 127.015 105.41) (width 0.762) (layer "B.Cu") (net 1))
 (segment (start 126.365 100.965) (end 127.015 101.615) (width 0.762) (layer "B.Cu") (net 1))
 (segment (start 134.62 98.425) (end 125.095 88.9) (width 0.762) (layer "B.Cu") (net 1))
 (segment (start 121.92 88.9) (end 120.015 90.805) (width 0.762) (layer "B.Cu") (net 1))
 (segment (start 123.19 100.965) (end 126.365 100.965) (width 0.762) (layer "B.Cu") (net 1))
 (segment (start 130.89 109.22) (end 130.89 112.395) (width 0.762) (layer "B.Cu") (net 1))
 (segment (start 120.055 120.65) (end 128.765 120.65) (width 0.762) (layer "F.Cu") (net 9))
 (segment (start 115.57 96.52) (end 115.57 118.11) (width 0.762) (layer "F.Cu") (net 9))
 (segment (start 104.394 83.44) (end 104.394 85.344) (width 0.762) (layer "F.Cu") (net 9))
 (segment (start 118.11 120.65) (end 120.055 120.65) (width 0.762) (layer "F.Cu") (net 9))
 (segment (start 115.57 118.11) (end 118.11 120.65) (width 0.762) (layer "F.Cu") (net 9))
 (segment (start 104.394 85.344) (end 115.57 96.52) (width 0.762) (layer "F.Cu") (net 9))
 (segment (start 132.715 90.17) (end 132.715 92.345) (width 0.762) (layer "F.Cu") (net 9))
 (via (at 132.715 90.17) (size 0.8) (drill 0.4) (layers "F.Cu" "B.Cu") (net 9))
 (segment (start 104.394 83.44) (end 125.985 83.44) (width 0.762) (layer "B.Cu") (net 9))
 (segment (start 125.985 83.44) (end 132.715 90.17) (width 0.762) (layer "B.Cu") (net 9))
 (segment (start 125.095 88.265) (end 119.38 88.265) (width 0.762) (layer "F.Cu") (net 10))
 (segment (start 130.42 81.28) (end 130.42 82.94) (width 0.762) (layer "F.Cu") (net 10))
 (segment (start 117.974 85.226) (end 116.84 86.36) (width 0.762) (layer "F.Cu") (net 10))
 (segment (start 125.73 87.63) (end 125.095 88.265) (width 0.762) (layer "F.Cu") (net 10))
 (segment (start 130.42 82.94) (end 125.73 87.63) (width 0.762) (layer "F.Cu") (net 10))
 (segment (start 117.974 81.28) (end 117.974 85.226) (width 0.762) (layer "F.Cu") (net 10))
 (via (at 119.38 88.265) (size 0.8) (drill 0.4) (layers "F.Cu" "B.Cu") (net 10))
 (via (at 116.84 86.36) (size 0.8) (drill 0.4) (layers "F.Cu" "B.Cu") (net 10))
 (segment (start 119.38 88.265) (end 113.03 94.615) (width 0.762) (layer "B.Cu") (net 10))
 (segment (start 113.03 94.615) (end 104.085 94.615) (width 0.762) (layer "B.Cu") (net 10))
 (segment (start 104.085 94.615) (end 101.53 92.06) (width 0.762) (layer "B.Cu") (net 10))
 (segment (start 111.14 92.06) (end 101.53 92.06) (width 0.762) (layer "B.Cu") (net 10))
 (segment (start 116.84 86.36) (end 111.14 92.06) (width 0.762) (layer "B.Cu") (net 10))
 (segment (start 113.674 71.619) (end 113.674 81.28) (width 0.762) (layer "F.Cu") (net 7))
 (segment (start 114.808 70.485) (end 113.674 71.619) (width 0.762) (layer "F.Cu") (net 7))
 (segment (start 126.12 71.619) (end 126.12 81.28) (width 0.762) (layer "F.Cu") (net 11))
 (segment (start 127.254 70.485) (end 126.12 71.619) (width 0.762) (layer "F.Cu") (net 11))
 (segment (start 186.69 105.41) (end 196.85 115.57) (width 0.762) (layer "F.Cu") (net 2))
 (segment (start 167.005 105.425) (end 174.61 105.425) (width 0.762) (layer "F.Cu") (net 2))
 (segment (start 196.85 115.57) (end 199.115 115.57) (width 0.762) (layer "F.Cu") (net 2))
 (segment (start 174.61 105.425) (end 174.625 105.41) (width 0.762) (layer "F.Cu") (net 2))
 (segment (start 179.705 105.41) (end 186.69 105.41) (width 0.762) (layer "F.Cu") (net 2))
 (segment (start 174.625 105.41) (end 175.26 105.41) (width 0.762) (layer "F.Cu") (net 2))
 (via (at 179.705 105.41) (size 0.8) (drill 0.4) (layers "F.Cu" "B.Cu") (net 2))
 (via (at 175.26 105.41) (size 0.8) (drill 0.4) (layers "F.Cu" "B.Cu") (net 2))
 (segment (start 175.26 105.41) (end 179.07 105.41) (width 0.762) (layer "B.Cu") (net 2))
 (segment (start 179.07 105.41) (end 179.705 105.41) (width 0.762) (layer "B.Cu") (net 2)))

